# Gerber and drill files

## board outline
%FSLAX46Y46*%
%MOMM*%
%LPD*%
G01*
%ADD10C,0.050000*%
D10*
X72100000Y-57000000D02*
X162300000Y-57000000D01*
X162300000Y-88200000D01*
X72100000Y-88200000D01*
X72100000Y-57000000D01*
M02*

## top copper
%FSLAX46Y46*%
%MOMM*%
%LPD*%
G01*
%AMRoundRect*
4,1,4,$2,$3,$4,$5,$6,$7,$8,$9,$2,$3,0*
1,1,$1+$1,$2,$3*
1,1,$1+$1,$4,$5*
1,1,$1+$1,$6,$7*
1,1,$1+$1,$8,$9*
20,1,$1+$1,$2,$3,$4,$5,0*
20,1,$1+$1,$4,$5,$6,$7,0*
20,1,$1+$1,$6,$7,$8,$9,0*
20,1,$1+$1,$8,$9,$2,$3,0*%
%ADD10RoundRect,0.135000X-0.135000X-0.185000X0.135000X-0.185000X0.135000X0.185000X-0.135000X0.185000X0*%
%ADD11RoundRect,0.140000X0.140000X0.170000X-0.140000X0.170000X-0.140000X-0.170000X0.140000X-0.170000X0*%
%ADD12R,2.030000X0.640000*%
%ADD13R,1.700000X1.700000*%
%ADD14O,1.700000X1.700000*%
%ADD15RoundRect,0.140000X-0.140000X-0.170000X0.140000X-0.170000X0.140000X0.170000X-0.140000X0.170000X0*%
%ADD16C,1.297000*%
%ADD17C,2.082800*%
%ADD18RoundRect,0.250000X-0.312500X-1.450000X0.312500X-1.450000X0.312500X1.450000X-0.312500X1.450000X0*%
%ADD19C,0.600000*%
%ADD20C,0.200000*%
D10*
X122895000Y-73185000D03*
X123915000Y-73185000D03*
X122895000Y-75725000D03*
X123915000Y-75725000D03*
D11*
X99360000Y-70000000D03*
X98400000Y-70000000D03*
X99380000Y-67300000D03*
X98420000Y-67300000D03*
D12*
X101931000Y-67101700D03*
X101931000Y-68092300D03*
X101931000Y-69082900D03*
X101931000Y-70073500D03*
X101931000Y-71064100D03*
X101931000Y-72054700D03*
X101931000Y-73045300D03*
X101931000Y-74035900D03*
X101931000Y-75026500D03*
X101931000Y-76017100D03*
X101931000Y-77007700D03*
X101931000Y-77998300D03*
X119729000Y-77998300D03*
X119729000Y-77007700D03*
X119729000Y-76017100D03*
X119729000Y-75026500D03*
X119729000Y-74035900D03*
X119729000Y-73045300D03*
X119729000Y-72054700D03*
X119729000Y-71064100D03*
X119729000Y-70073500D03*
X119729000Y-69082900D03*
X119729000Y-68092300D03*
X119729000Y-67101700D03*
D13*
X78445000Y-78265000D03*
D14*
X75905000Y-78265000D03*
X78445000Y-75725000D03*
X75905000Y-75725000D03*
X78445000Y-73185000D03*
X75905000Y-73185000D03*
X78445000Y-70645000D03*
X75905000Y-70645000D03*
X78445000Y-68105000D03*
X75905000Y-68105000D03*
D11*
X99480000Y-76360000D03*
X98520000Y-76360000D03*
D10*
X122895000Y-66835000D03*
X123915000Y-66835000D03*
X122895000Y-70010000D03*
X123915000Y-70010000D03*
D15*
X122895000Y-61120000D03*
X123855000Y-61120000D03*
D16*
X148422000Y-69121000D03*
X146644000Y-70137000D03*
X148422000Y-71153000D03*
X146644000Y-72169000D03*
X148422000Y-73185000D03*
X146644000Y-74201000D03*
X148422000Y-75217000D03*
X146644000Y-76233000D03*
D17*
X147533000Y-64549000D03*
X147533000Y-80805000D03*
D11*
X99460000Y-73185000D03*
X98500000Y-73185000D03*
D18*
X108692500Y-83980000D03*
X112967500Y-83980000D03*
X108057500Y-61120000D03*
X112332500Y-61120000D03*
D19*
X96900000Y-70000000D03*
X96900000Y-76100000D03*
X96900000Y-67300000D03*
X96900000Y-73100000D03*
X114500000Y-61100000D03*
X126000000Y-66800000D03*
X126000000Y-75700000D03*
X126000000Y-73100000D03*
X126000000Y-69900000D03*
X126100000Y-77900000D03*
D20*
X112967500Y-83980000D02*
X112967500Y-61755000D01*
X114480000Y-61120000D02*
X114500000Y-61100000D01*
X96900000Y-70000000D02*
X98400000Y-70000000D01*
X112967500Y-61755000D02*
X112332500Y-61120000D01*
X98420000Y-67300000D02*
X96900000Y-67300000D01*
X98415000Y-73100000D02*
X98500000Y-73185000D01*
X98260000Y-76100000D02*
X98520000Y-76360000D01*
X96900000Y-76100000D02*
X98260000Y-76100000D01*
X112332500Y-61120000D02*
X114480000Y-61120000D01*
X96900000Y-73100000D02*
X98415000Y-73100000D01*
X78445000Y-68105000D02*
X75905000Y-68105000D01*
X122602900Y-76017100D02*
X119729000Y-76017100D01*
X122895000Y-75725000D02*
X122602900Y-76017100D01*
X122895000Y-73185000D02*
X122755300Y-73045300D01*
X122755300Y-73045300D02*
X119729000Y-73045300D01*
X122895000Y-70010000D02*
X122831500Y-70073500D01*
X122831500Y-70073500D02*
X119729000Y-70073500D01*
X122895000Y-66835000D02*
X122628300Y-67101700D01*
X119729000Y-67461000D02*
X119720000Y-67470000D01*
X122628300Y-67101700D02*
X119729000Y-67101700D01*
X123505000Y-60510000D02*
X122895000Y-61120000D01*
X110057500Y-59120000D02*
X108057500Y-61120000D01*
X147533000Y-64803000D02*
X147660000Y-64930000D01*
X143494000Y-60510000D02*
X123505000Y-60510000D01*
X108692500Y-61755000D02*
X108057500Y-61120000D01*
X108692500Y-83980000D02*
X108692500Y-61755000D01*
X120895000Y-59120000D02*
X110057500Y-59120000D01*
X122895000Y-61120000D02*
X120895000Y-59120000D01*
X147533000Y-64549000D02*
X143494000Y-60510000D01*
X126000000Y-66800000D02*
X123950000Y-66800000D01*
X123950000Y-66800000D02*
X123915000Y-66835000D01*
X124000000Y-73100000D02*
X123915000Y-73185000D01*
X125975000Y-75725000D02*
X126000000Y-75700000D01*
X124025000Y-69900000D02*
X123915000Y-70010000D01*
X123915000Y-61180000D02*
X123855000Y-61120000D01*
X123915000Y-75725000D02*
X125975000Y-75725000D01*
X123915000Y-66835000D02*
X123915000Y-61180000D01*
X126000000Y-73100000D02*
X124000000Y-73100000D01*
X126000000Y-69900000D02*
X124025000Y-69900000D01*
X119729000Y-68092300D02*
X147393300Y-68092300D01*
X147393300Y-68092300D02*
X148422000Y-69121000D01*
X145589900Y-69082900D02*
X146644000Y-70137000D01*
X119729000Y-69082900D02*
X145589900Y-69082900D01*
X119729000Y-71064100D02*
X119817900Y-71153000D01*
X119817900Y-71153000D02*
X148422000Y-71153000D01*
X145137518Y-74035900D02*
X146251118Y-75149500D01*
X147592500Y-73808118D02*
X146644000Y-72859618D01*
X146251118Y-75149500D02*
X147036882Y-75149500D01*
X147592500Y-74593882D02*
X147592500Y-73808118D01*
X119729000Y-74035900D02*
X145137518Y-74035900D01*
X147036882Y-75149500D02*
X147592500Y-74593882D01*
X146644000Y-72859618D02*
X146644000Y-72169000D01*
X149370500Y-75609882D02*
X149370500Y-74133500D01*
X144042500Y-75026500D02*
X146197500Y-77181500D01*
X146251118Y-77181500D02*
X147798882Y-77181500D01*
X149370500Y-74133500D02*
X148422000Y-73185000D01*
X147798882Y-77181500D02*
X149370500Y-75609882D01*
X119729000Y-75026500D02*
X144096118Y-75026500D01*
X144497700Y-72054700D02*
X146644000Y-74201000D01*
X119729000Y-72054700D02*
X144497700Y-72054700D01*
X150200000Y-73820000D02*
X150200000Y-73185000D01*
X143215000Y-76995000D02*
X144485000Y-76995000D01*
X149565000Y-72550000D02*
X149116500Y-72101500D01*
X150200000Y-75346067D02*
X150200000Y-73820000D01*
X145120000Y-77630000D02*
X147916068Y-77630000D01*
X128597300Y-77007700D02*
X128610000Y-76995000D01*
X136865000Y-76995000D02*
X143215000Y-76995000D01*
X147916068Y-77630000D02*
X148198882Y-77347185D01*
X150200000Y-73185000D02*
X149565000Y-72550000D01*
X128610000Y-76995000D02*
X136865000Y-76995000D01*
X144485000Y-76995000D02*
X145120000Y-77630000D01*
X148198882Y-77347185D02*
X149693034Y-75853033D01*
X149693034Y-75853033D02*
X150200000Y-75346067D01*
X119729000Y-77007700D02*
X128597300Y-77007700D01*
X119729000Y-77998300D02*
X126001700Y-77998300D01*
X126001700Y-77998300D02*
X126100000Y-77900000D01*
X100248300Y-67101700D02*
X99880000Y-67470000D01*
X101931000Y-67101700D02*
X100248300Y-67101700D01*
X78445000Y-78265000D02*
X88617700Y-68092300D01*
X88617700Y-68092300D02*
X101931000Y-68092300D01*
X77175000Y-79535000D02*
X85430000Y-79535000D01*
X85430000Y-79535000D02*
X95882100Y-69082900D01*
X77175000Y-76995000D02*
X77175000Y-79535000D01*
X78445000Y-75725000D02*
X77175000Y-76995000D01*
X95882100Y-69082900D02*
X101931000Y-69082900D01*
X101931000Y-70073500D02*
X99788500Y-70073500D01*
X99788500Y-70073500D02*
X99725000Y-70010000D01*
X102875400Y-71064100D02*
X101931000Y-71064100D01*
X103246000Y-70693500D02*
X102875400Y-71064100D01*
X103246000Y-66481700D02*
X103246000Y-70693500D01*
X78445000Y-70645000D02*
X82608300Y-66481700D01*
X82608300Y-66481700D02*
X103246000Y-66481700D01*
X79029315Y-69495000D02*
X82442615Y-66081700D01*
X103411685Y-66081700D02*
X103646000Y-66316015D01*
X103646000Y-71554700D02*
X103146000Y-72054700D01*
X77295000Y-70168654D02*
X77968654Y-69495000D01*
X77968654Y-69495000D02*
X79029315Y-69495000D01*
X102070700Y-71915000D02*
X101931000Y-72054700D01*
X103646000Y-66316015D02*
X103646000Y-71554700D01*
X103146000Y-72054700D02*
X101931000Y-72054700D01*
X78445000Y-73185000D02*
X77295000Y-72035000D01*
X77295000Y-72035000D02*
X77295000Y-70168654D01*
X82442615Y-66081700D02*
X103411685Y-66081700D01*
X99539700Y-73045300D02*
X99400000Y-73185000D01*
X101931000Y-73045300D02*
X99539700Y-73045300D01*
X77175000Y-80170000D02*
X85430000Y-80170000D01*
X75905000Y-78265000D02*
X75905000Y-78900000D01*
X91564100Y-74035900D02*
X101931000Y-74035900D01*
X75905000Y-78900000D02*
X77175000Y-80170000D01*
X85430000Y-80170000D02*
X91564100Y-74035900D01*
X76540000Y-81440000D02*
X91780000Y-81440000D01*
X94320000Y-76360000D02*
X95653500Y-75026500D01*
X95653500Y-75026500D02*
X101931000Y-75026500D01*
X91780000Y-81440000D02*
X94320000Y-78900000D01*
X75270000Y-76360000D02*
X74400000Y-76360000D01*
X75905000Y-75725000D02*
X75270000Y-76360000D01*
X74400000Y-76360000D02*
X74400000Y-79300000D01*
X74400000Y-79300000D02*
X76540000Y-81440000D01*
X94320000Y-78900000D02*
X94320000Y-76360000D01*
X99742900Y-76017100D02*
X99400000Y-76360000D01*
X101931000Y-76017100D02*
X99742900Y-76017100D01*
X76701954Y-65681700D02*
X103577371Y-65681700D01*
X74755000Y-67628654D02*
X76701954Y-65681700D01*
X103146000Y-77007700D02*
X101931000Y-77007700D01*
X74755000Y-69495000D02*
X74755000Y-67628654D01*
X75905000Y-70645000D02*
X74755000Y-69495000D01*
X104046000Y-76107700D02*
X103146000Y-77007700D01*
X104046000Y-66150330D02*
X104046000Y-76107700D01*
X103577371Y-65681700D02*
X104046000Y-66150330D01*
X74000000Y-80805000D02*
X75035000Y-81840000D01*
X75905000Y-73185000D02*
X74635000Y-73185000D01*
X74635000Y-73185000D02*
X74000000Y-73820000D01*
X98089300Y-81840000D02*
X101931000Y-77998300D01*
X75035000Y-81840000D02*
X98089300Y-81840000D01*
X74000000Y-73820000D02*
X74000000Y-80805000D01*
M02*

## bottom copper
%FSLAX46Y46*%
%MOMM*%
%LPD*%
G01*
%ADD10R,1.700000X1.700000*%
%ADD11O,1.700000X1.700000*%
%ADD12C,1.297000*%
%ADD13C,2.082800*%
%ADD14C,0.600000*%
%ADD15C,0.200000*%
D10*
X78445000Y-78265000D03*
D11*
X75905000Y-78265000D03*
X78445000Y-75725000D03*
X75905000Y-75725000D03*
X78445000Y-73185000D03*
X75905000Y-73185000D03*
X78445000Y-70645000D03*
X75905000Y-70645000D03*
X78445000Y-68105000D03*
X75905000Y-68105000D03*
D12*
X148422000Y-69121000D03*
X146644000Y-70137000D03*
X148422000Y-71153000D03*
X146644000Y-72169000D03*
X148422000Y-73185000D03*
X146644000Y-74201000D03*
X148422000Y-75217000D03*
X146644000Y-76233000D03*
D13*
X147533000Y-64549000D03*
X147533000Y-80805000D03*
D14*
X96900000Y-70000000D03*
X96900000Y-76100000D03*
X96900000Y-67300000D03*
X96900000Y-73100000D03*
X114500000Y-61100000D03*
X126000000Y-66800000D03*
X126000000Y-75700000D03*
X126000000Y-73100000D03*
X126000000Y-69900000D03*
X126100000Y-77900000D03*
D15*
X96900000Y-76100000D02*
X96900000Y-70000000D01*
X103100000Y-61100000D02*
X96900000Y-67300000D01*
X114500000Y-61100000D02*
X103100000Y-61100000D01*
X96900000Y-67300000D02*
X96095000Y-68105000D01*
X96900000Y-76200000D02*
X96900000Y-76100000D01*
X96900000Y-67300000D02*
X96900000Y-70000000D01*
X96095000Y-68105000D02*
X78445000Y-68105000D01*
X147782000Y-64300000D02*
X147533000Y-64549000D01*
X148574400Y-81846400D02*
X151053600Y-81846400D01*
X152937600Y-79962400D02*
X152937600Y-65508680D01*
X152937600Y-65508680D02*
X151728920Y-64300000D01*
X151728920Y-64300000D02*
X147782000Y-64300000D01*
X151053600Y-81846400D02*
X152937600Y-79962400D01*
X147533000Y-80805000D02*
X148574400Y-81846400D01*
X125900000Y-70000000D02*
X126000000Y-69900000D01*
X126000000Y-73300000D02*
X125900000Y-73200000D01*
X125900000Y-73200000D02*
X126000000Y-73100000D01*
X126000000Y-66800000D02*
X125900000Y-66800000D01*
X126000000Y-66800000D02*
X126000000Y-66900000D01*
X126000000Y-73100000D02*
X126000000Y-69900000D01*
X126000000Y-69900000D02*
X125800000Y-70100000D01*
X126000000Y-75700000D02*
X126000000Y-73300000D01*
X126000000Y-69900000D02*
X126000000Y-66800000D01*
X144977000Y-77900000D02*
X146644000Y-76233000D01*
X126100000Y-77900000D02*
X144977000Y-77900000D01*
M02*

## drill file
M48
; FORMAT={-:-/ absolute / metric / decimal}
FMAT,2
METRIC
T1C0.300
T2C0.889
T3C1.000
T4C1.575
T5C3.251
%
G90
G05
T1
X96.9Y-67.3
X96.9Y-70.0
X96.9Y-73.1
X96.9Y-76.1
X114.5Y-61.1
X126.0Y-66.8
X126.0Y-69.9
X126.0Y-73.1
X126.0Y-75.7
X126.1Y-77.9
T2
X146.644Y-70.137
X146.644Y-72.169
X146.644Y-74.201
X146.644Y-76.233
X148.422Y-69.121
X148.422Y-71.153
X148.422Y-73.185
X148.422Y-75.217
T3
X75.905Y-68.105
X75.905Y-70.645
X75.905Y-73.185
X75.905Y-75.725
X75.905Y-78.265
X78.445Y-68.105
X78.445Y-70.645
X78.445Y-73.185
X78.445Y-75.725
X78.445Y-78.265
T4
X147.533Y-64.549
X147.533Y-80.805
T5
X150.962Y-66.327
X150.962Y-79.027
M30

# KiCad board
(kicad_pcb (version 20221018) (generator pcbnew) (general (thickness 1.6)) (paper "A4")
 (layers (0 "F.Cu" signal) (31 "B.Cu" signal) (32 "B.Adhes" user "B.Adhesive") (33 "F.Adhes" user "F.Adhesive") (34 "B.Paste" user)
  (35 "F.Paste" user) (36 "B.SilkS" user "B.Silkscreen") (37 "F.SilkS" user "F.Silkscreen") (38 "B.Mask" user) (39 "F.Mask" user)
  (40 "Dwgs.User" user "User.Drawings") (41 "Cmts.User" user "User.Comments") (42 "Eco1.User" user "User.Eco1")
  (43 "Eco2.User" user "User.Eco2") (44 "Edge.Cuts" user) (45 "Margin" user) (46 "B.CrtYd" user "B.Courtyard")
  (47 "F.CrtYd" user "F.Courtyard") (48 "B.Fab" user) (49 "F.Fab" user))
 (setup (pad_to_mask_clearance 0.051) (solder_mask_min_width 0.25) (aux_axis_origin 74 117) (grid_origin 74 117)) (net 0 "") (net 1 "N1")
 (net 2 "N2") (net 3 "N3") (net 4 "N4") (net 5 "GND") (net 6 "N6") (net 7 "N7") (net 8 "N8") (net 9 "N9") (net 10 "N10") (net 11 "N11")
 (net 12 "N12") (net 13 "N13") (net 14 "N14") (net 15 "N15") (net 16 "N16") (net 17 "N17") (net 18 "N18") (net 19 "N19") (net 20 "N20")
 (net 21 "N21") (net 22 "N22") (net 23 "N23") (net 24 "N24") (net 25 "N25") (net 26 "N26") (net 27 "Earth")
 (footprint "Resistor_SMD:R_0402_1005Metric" (layer "F.Cu") (at 123.405 73.185)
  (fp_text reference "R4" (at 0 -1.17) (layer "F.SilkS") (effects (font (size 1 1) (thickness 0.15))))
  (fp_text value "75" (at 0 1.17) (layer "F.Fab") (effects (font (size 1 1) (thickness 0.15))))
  (pad "1" smd roundrect (at -0.51 0) (size 0.54 0.64) (layers "F.Cu" "F.Paste" "F.Mask") (roundrect_rratio 0.25) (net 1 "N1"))
  (pad "2" smd roundrect (at 0.51 0) (size 0.54 0.64) (layers "F.Cu" "F.Paste" "F.Mask") (roundrect_rratio 0.25) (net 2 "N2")))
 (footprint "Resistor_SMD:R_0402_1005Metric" (layer "F.Cu") (at 123.405 75.725)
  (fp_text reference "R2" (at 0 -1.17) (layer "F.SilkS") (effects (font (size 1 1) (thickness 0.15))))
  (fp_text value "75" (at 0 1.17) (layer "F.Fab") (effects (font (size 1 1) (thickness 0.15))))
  (pad "1" smd roundrect (at -0.51 0) (size 0.54 0.64) (layers "F.Cu" "F.Paste" "F.Mask") (roundrect_rratio 0.25) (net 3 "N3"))
  (pad "2" smd roundrect (at 0.51 0) (size 0.54 0.64) (layers "F.Cu" "F.Paste" "F.Mask") (roundrect_rratio 0.25) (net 2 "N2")))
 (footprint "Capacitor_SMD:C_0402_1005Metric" (layer "F.Cu") (at 98.88 70 180)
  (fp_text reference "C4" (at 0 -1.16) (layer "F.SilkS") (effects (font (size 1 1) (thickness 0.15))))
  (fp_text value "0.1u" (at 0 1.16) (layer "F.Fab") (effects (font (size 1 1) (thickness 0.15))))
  (pad "1" smd roundrect (at -0.48 0 180) (size 0.56 0.62) (layers "F.Cu" "F.Paste" "F.Mask") (roundrect_rratio 0.25) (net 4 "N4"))
  (pad "2" smd roundrect (at 0.48 0 180) (size 0.56 0.62) (layers "F.Cu" "F.Paste" "F.Mask") (roundrect_rratio 0.25) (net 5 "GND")))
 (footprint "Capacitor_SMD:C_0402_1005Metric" (layer "F.Cu") (at 98.9 67.3 180)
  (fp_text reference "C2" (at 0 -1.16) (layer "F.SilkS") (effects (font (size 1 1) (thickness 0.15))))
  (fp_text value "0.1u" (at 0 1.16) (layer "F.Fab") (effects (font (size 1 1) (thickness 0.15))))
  (pad "1" smd roundrect (at -0.48 0 180) (size 0.56 0.62) (layers "F.Cu" "F.Paste" "F.Mask") (roundrect_rratio 0.25) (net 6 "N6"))
  (pad "2" smd roundrect (at 0.48 0 180) (size 0.56 0.62) (layers "F.Cu" "F.Paste" "F.Mask") (roundrect_rratio 0.25) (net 5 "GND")))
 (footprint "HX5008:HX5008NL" (layer "F.Cu") (at 106.63 72.55)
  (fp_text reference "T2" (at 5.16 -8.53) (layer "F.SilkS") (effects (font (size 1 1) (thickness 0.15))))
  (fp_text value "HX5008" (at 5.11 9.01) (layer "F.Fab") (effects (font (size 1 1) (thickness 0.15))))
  (pad "1" smd rect (at -4.699 -5.4483 270) (size 0.64 2.03) (layers "F.Cu" "F.Paste" "F.Mask") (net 6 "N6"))
  (pad "2" smd rect (at -4.699 -4.4577 270) (size 0.64 2.03) (layers "F.Cu" "F.Paste" "F.Mask") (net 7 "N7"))
  (pad "3" smd rect (at -4.699 -3.4671 270) (size 0.64 2.03) (layers "F.Cu" "F.Paste" "F.Mask") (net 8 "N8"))
  (pad "4" smd rect (at -4.699 -2.4765 270) (size 0.64 2.03) (layers "F.Cu" "F.Paste" "F.Mask") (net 4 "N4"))
  (pad "5" smd rect (at -4.699 -1.4859 270) (size 0.64 2.03) (layers "F.Cu" "F.Paste" "F.Mask") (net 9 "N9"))
  (pad "6" smd rect (at -4.699 -0.4953 270) (size 0.64 2.03) (layers "F.Cu" "F.Paste" "F.Mask") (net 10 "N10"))
  (pad "7" smd rect (at -4.699 0.4953 270) (size 0.64 2.03) (layers "F.Cu" "F.Paste" "F.Mask") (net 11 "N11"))
  (pad "8" smd rect (at -4.699 1.4859 270) (size 0.64 2.03) (layers "F.Cu" "F.Paste" "F.Mask") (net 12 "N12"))
  (pad "9" smd rect (at -4.699 2.4765 270) (size 0.64 2.03) (layers "F.Cu" "F.Paste" "F.Mask") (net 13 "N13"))
  (pad "10" smd rect (at -4.699 3.4671 270) (size 0.64 2.03) (layers "F.Cu" "F.Paste" "F.Mask") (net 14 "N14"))
  (pad "11" smd rect (at -4.699 4.4577 270) (size 0.64 2.03) (layers "F.Cu" "F.Paste" "F.Mask") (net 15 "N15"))
  (pad "12" smd rect (at -4.699 5.4483 270) (size 0.64 2.03) (layers "F.Cu" "F.Paste" "F.Mask") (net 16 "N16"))
  (pad "13" smd rect (at 13.099 5.4483 270) (size 0.64 2.03) (layers "F.Cu" "F.Paste" "F.Mask") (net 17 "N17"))
  (pad "14" smd rect (at 13.099 4.4577 270) (size 0.64 2.03) (layers "F.Cu" "F.Paste" "F.Mask") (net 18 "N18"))
  (pad "15" smd rect (at 13.099 3.4671 270) (size 0.64 2.03) (layers "F.Cu" "F.Paste" "F.Mask") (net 3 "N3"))
  (pad "16" smd rect (at 13.099 2.4765 270) (size 0.64 2.03) (layers "F.Cu" "F.Paste" "F.Mask") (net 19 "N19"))
  (pad "17" smd rect (at 13.099 1.4859 270) (size 0.64 2.03) (layers "F.Cu" "F.Paste" "F.Mask") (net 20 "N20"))
  (pad "18" smd rect (at 13.099 0.4953 270) (size 0.64 2.03) (layers "F.Cu" "F.Paste" "F.Mask") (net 1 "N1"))
  (pad "19" smd rect (at 13.099 -0.4953 270) (size 0.64 2.03) (layers "F.Cu" "F.Paste" "F.Mask") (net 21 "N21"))
  (pad "20" smd rect (at 13.099 -1.4859 270) (size 0.64 2.03) (layers "F.Cu" "F.Paste" "F.Mask") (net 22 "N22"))
  (pad "21" smd rect (at 13.099 -2.4765 270) (size 0.64 2.03) (layers "F.Cu" "F.Paste" "F.Mask") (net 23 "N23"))
  (pad "22" smd rect (at 13.099 -3.4671 270) (size 0.64 2.03) (layers "F.Cu" "F.Paste" "F.Mask") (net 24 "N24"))
  (pad "23" smd rect (at 13.099 -4.4577 270) (size 0.64 2.03) (layers "F.Cu" "F.Paste" "F.Mask") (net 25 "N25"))
  (pad "24" smd rect (at 13.099 -5.4483 270) (size 0.64 2.03) (layers "F.Cu" "F.Paste" "F.Mask") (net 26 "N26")))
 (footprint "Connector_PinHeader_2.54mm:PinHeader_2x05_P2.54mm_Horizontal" (layer "F.Cu") (at 78.445 78.265 180)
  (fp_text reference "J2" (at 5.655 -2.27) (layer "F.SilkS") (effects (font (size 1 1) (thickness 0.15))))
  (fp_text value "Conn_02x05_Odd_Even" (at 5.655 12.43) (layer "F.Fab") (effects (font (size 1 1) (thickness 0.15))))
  (pad "1" thru_hole rect (at 0 0 180) (size 1.7 1.7) (drill 1) (layers "*.Cu" "*.Mask") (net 7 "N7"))
  (pad "2" thru_hole oval (at 2.54 0 180) (size 1.7 1.7) (drill 1) (layers "*.Cu" "*.Mask") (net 12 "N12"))
  (pad "3" thru_hole oval (at 0 2.54 180) (size 1.7 1.7) (drill 1) (layers "*.Cu" "*.Mask") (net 8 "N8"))
  (pad "4" thru_hole oval (at 2.54 2.54 180) (size 1.7 1.7) (drill 1) (layers "*.Cu" "*.Mask") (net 13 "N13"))
  (pad "5" thru_hole oval (at 0 5.08 180) (size 1.7 1.7) (drill 1) (layers "*.Cu" "*.Mask") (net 10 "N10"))
  (pad "6" thru_hole oval (at 2.54 5.08 180) (size 1.7 1.7) (drill 1) (layers "*.Cu" "*.Mask") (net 16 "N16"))
  (pad "7" thru_hole oval (at 0 7.62 180) (size 1.7 1.7) (drill 1) (layers "*.Cu" "*.Mask") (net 9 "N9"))
  (pad "8" thru_hole oval (at 2.54 7.62 180) (size 1.7 1.7) (drill 1) (layers "*.Cu" "*.Mask") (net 15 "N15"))
  (pad "9" thru_hole oval (at 0 10.16 180) (size 1.7 1.7) (drill 1) (layers "*.Cu" "*.Mask") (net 5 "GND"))
  (pad "10" thru_hole oval (at 2.54 10.16 180) (size 1.7 1.7) (drill 1) (layers "*.Cu" "*.Mask") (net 5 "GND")))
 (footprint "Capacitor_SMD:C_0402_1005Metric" (layer "F.Cu") (at 99 76.36 180)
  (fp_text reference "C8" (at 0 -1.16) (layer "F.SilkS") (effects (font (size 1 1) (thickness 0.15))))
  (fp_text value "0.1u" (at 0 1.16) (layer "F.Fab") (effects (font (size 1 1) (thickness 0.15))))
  (pad "1" smd roundrect (at -0.48 0 180) (size 0.56 0.62) (layers "F.Cu" "F.Paste" "F.Mask") (roundrect_rratio 0.25) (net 14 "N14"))
  (pad "2" smd roundrect (at 0.48 0 180) (size 0.56 0.62) (layers "F.Cu" "F.Paste" "F.Mask") (roundrect_rratio 0.25) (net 5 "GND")))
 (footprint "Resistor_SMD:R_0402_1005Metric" (layer "F.Cu") (at 123.405 66.835)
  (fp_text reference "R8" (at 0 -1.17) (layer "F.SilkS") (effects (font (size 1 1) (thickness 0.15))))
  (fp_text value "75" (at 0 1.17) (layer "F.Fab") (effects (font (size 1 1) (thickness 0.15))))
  (pad "1" smd roundrect (at -0.51 0) (size 0.54 0.64) (layers "F.Cu" "F.Paste" "F.Mask") (roundrect_rratio 0.25) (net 26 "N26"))
  (pad "2" smd roundrect (at 0.51 0) (size 0.54 0.64) (layers "F.Cu" "F.Paste" "F.Mask") (roundrect_rratio 0.25) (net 2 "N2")))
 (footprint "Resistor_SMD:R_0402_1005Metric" (layer "F.Cu") (at 123.405 70.01)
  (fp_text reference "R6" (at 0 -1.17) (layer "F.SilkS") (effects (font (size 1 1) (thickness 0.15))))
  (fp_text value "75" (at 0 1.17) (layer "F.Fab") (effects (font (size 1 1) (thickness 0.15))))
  (pad "1" smd roundrect (at -0.51 0) (size 0.54 0.64) (layers "F.Cu" "F.Paste" "F.Mask") (roundrect_rratio 0.25) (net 23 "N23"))
  (pad "2" smd roundrect (at 0.51 0) (size 0.54 0.64) (layers "F.Cu" "F.Paste" "F.Mask") (roundrect_rratio 0.25) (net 2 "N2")))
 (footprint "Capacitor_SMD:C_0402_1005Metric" (layer "F.Cu") (at 123.375 61.12)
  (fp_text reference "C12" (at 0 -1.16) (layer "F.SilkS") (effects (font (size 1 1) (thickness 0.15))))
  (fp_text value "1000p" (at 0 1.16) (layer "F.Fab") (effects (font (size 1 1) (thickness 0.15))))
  (pad "1" smd roundrect (at -0.48 0) (size 0.56 0.62) (layers "F.Cu" "F.Paste" "F.Mask") (roundrect_rratio 0.25) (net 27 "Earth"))
  (pad "2" smd roundrect (at 0.48 0) (size 0.56 0.62) (layers "F.Cu" "F.Paste" "F.Mask") (roundrect_rratio 0.25) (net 2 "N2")))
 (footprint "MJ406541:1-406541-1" (layer "F.Cu") (at 148.422 69.121 -90)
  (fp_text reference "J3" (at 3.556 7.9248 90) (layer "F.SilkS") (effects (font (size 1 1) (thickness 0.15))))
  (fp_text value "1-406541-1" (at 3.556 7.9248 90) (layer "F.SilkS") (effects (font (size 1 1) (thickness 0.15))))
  (pad "" np_thru_hole circle (at -2.794 -2.54 270) (size 3.2512 3.2512) (drill 3.2512) (layers "*.Cu" "*.Mask"))
  (pad "" np_thru_hole circle (at 9.906 -2.54 270) (size 3.2512 3.2512) (drill 3.2512) (layers "*.Cu" "*.Mask"))
  (pad "1" thru_hole circle (at 0 0 270) (size 1.297 1.297) (drill 0.889) (layers "*.Cu" "*.Mask") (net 25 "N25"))
  (pad "2" thru_hole circle (at 1.016 1.778 270) (size 1.297 1.297) (drill 0.889) (layers "*.Cu" "*.Mask") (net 24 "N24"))
  (pad "3" thru_hole circle (at 2.032 0 270) (size 1.297 1.297) (drill 0.889) (layers "*.Cu" "*.Mask") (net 22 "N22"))
  (pad "4" thru_hole circle (at 3.048 1.778 270) (size 1.297 1.297) (drill 0.889) (layers "*.Cu" "*.Mask") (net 20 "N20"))
  (pad "5" thru_hole circle (at 4.064 0 270) (size 1.297 1.297) (drill 0.889) (layers "*.Cu" "*.Mask") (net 19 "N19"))
  (pad "6" thru_hole circle (at 5.08 1.778 270) (size 1.297 1.297) (drill 0.889) (layers "*.Cu" "*.Mask") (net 21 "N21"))
  (pad "7" thru_hole circle (at 6.096 0 270) (size 1.297 1.297) (drill 0.889) (layers "*.Cu" "*.Mask") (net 18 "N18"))
  (pad "8" thru_hole circle (at 7.112 1.778 270) (size 1.297 1.297) (drill 0.889) (layers "*.Cu" "*.Mask") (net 17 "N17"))
  (pad "9" thru_hole circle (at -4.572 0.889 270) (size 2.0828 2.0828) (drill 1.5748) (layers "*.Cu" "*.Mask") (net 27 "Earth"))
  (pad "10" thru_hole circle (at 11.684 0.889 270) (size 2.0828 2.0828) (drill 1.5748) (layers "*.Cu" "*.Mask") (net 27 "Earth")))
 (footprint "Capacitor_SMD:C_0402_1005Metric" (layer "F.Cu") (at 98.98 73.185 180)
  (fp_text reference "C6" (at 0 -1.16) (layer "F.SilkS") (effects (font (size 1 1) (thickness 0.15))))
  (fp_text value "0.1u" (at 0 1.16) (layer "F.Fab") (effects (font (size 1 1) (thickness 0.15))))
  (pad "1" smd roundrect (at -0.48 0 180) (size 0.56 0.62) (layers "F.Cu" "F.Paste" "F.Mask") (roundrect_rratio 0.25) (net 11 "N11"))
  (pad "2" smd roundrect (at 0.48 0 180) (size 0.56 0.62) (layers "F.Cu" "F.Paste" "F.Mask") (roundrect_rratio 0.25) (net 5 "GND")))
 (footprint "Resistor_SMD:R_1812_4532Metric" (layer "F.Cu") (at 110.83 83.98)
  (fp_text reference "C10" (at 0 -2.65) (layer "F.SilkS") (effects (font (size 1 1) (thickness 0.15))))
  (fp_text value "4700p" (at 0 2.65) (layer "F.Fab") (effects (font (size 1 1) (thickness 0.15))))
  (pad "1" smd roundrect (at -2.1375 0) (size 1.125 3.4) (layers "F.Cu" "F.Paste" "F.Mask") (roundrect_rratio 0.222222) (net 27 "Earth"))
  (pad "2" smd roundrect (at 2.1375 0) (size 1.125 3.4) (layers "F.Cu" "F.Paste" "F.Mask") (roundrect_rratio 0.222222) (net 5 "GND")))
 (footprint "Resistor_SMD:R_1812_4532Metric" (layer "F.Cu") (at 110.195 61.12)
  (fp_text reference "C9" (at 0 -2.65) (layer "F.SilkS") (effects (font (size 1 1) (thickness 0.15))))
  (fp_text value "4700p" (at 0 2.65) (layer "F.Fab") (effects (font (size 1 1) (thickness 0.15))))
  (pad "1" smd roundrect (at -2.1375 0) (size 1.125 3.4) (layers "F.Cu" "F.Paste" "F.Mask") (roundrect_rratio 0.222222) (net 27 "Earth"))
  (pad "2" smd roundrect (at 2.1375 0) (size 1.125 3.4) (layers "F.Cu" "F.Paste" "F.Mask") (roundrect_rratio 0.222222) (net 5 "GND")))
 (gr_rect (start 72.1 57) (end 162.3 88.2) (stroke (width 0.05) (type default)) (fill none) (layer "Edge.Cuts"))
 (segment (start 112.9675 83.98) (end 112.9675 61.755) (width 0.2) (layer "F.Cu") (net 5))
 (segment (start 114.48 61.12) (end 114.5 61.1) (width 0.2) (layer "F.Cu") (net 5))
 (segment (start 96.9 70) (end 98.4 70) (width 0.2) (layer "F.Cu") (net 5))
 (segment (start 112.9675 61.755) (end 112.3325 61.12) (width 0.2) (layer "F.Cu") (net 5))
 (segment (start 98.42 67.3) (end 96.9 67.3) (width 0.2) (layer "F.Cu") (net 5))
 (segment (start 98.415 73.1) (end 98.5 73.185) (width 0.2) (layer "F.Cu") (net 5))
 (segment (start 98.26 76.1) (end 98.52 76.36) (width 0.2) (layer "F.Cu") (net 5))
 (segment (start 96.9 76.1) (end 98.26 76.1) (width 0.2) (layer "F.Cu") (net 5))
 (segment (start 112.3325 61.12) (end 114.48 61.12) (width 0.2) (layer "F.Cu") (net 5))
 (segment (start 96.9 73.1) (end 98.415 73.1) (width 0.2) (layer "F.Cu") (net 5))
 (segment (start 78.445 68.105) (end 75.905 68.105) (width 0.2) (layer "F.Cu") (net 5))
 (via (at 96.9 70) (size 0.6) (drill 0.3) (layers "F.Cu" "B.Cu") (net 5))
 (via (at 96.9 76.1) (size 0.6) (drill 0.3) (layers "F.Cu" "B.Cu") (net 5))
 (via (at 96.9 67.3) (size 0.6) (drill 0.3) (layers "F.Cu" "B.Cu") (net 5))
 (via (at 96.9 73.1) (size 0.6) (drill 0.3) (layers "F.Cu" "B.Cu") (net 5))
 (via (at 114.5 61.1) (size 0.6) (drill 0.3) (layers "F.Cu" "B.Cu") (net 5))
 (segment (start 96.9 76.1) (end 96.9 70) (width 0.2) (layer "B.Cu") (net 5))
 (segment (start 103.1 61.1) (end 96.9 67.3) (width 0.2) (layer "B.Cu") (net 5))
 (segment (start 114.5 61.1) (end 103.1 61.1) (width 0.2) (layer "B.Cu") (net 5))
 (segment (start 96.9 67.3) (end 96.095 68.105) (width 0.2) (layer "B.Cu") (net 5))
 (segment (start 96.9 76.2) (end 96.9 76.1) (width 0.2) (layer "B.Cu") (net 5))
 (segment (start 96.9 67.3) (end 96.9 70) (width 0.2) (layer "B.Cu") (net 5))
 (segment (start 96.095 68.105) (end 78.445 68.105) (width 0.2) (layer "B.Cu") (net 5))
 (segment (start 122.6029 76.0171) (end 119.729 76.0171) (width 0.2) (layer "F.Cu") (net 3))
 (segment (start 122.895 75.725) (end 122.6029 76.0171) (width 0.2) (layer "F.Cu") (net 3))
 (segment (start 122.895 73.185) (end 122.7553 73.0453) (width 0.2) (layer "F.Cu") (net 1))
 (segment (start 122.7553 73.0453) (end 119.729 73.0453) (width 0.2) (layer "F.Cu") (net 1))
 (segment (start 122.895 70.01) (end 122.8315 70.0735) (width 0.2) (layer "F.Cu") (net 23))
 (segment (start 122.8315 70.0735) (end 119.729 70.0735) (width 0.2) (layer "F.Cu") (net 23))
 (segment (start 122.895 66.835) (end 122.6283 67.1017) (width 0.2) (layer "F.Cu") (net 26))
 (segment (start 119.729 67.461) (end 119.72 67.47) (width 0.2) (layer "F.Cu") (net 26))
 (segment (start 122.6283 67.1017) (end 119.729 67.1017) (width 0.2) (layer "F.Cu") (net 26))
 (segment (start 123.505 60.51) (end 122.895 61.12) (width 0.2) (layer "F.Cu") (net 27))
 (segment (start 110.0575 59.12) (end 108.0575 61.12) (width 0.2) (layer "F.Cu") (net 27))
 (segment (start 147.533 64.803) (end 147.66 64.93) (width 0.2) (layer "F.Cu") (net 27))
 (segment (start 143.494 60.51) (end 123.505 60.51) (width 0.2) (layer "F.Cu") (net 27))
 (segment (start 108.6925 61.755) (end 108.0575 61.12) (width 0.2) (layer "F.Cu") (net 27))
 (segment (start 108.6925 83.98) (end 108.6925 61.755) (width 0.2) (layer "F.Cu") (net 27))
 (segment (start 120.895 59.12) (end 110.0575 59.12) (width 0.2) (layer "F.Cu") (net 27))
 (segment (start 122.895 61.12) (end 120.895 59.12) (width 0.2) (layer "F.Cu") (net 27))
 (segment (start 147.533 64.549) (end 143.494 60.51) (width 0.2) (layer "F.Cu") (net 27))
 (segment (start 147.782 64.3) (end 147.533 64.549) (width 0.2) (layer "B.Cu") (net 27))
 (segment (start 148.5744 81.8464) (end 151.0536 81.8464) (width 0.2) (layer "B.Cu") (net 27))
 (segment (start 152.9376 79.9624) (end 152.9376 65.50868) (width 0.2) (layer "B.Cu") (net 27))
 (segment (start 152.9376 65.50868) (end 151.72892 64.3) (width 0.2) (layer "B.Cu") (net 27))
 (segment (start 151.72892 64.3) (end 147.782 64.3) (width 0.2) (layer "B.Cu") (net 27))
 (segment (start 151.0536 81.8464) (end 152.9376 79.9624) (width 0.2) (layer "B.Cu") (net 27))
 (segment (start 147.533 80.805) (end 148.5744 81.8464) (width 0.2) (layer "B.Cu") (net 27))
 (segment (start 126 66.8) (end 123.95 66.8) (width 0.2) (layer "F.Cu") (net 2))
 (segment (start 123.95 66.8) (end 123.915 66.835) (width 0.2) (layer "F.Cu") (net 2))
 (segment (start 124 73.1) (end 123.915 73.185) (width 0.2) (layer "F.Cu") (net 2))
 (segment (start 125.975 75.725) (end 126 75.7) (width 0.2) (layer "F.Cu") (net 2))
 (segment (start 124.025 69.9) (end 123.915 70.01) (width 0.2) (layer "F.Cu") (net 2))
 (segment (start 123.915 61.18) (end 123.855 61.12) (width 0.2) (layer "F.Cu") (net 2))
 (segment (start 123.915 75.725) (end 125.975 75.725) (width 0.2) (layer "F.Cu") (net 2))
 (segment (start 123.915 66.835) (end 123.915 61.18) (width 0.2) (layer "F.Cu") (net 2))
 (segment (start 126 73.1) (end 124 73.1) (width 0.2) (layer "F.Cu") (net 2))
 (segment (start 126 69.9) (end 124.025 69.9) (width 0.2) (layer "F.Cu") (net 2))
 (via (at 126 66.8) (size 0.6) (drill 0.3) (layers "F.Cu" "B.Cu") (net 2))
 (via (at 126 75.7) (size 0.6) (drill 0.3) (layers "F.Cu" "B.Cu") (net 2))
 (via (at 126 73.1) (size 0.6) (drill 0.3) (layers "F.Cu" "B.Cu") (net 2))
 (via (at 126 69.9) (size 0.6) (drill 0.3) (layers "F.Cu" "B.Cu") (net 2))
 (segment (start 125.9 70) (end 126 69.9) (width 0.2) (layer "B.Cu") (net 2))
 (segment (start 126 73.3) (end 125.9 73.2) (width 0.2) (layer "B.Cu") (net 2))
 (segment (start 125.9 73.2) (end 126 73.1) (width 0.2) (layer "B.Cu") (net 2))
 (segment (start 126 66.8) (end 125.9 66.8) (width 0.2) (layer "B.Cu") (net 2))
 (segment (start 126 66.8) (end 126 66.9) (width 0.2) (layer "B.Cu") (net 2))
 (segment (start 126 73.1) (end 126 69.9) (width 0.2) (layer "B.Cu") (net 2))
 (segment (start 126 69.9) (end 125.8 70.1) (width 0.2) (layer "B.Cu") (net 2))
 (segment (start 126 75.7) (end 126 73.3) (width 0.2) (layer "B.Cu") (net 2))
 (segment (start 126 69.9) (end 126 66.8) (width 0.2) (layer "B.Cu") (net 2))
 (segment (start 119.729 68.0923) (end 147.3933 68.0923) (width 0.2) (layer "F.Cu") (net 25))
 (segment (start 147.3933 68.0923) (end 148.422 69.121) (width 0.2) (layer "F.Cu") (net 25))
 (segment (start 145.5899 69.0829) (end 146.644 70.137) (width 0.2) (layer "F.Cu") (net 24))
 (segment (start 119.729 69.0829) (end 145.5899 69.0829) (width 0.2) (layer "F.Cu") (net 24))
 (segment (start 119.729 71.0641) (end 119.8179 71.153) (width 0.2) (layer "F.Cu") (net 22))
 (segment (start 119.8179 71.153) (end 148.422 71.153) (width 0.2) (layer "F.Cu") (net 22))
 (segment (start 145.137518 74.0359) (end 146.251118 75.1495) (width 0.2) (layer "F.Cu") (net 20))
 (segment (start 147.5925 73.808118) (end 146.644 72.859618) (width 0.2) (layer "F.Cu") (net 20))
 (segment (start 146.251118 75.1495) (end 147.036882 75.1495) (width 0.2) (layer "F.Cu") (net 20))
 (segment (start 147.5925 74.593882) (end 147.5925 73.808118) (width 0.2) (layer "F.Cu") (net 20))
 (segment (start 119.729 74.0359) (end 145.137518 74.0359) (width 0.2) (layer "F.Cu") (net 20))
 (segment (start 147.036882 75.1495) (end 147.5925 74.593882) (width 0.2) (layer "F.Cu") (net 20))
 (segment (start 146.644 72.859618) (end 146.644 72.169) (width 0.2) (layer "F.Cu") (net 20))
 (segment (start 149.3705 75.609882) (end 149.3705 74.1335) (width 0.2) (layer "F.Cu") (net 19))
 (segment (start 144.0425 75.0265) (end 146.1975 77.1815) (width 0.2) (layer "F.Cu") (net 19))
 (segment (start 146.251118 77.1815) (end 147.798882 77.1815) (width 0.2) (layer "F.Cu") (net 19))
 (segment (start 149.3705 74.1335) (end 148.422 73.185) (width 0.2) (layer "F.Cu") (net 19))
 (segment (start 147.798882 77.1815) (end 149.3705 75.609882) (width 0.2) (layer "F.Cu") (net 19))
 (segment (start 119.729 75.0265) (end 144.096118 75.0265) (width 0.2) (layer "F.Cu") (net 19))
 (segment (start 144.4977 72.0547) (end 146.644 74.201) (width 0.2) (layer "F.Cu") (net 21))
 (segment (start 119.729 72.0547) (end 144.4977 72.0547) (width 0.2) (layer "F.Cu") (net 21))
 (segment (start 150.2 73.82) (end 150.2 73.185) (width 0.2) (layer "F.Cu") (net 18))
 (segment (start 143.215 76.995) (end 144.485 76.995) (width 0.2) (layer "F.Cu") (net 18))
 (segment (start 149.565 72.55) (end 149.1165 72.1015) (width 0.2) (layer "F.Cu") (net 18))
 (segment (start 150.2 75.346067) (end 150.2 73.82) (width 0.2) (layer "F.Cu") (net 18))
 (segment (start 145.12 77.63) (end 147.916068 77.63) (width 0.2) (layer "F.Cu") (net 18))
 (segment (start 128.5973 77.0077) (end 128.61 76.995) (width 0.2) (layer "F.Cu") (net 18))
 (segment (start 136.865 76.995) (end 143.215 76.995) (width 0.2) (layer "F.Cu") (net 18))
 (segment (start 147.916068 77.63) (end 148.198882 77.347185) (width 0.2) (layer "F.Cu") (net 18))
 (segment (start 150.2 73.185) (end 149.565 72.55) (width 0.2) (layer "F.Cu") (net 18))
 (segment (start 128.61 76.995) (end 136.865 76.995) (width 0.2) (layer "F.Cu") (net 18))
 (segment (start 144.485 76.995) (end 145.12 77.63) (width 0.2) (layer "F.Cu") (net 18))
 (segment (start 148.198882 77.347185) (end 149.693034 75.853033) (width 0.2) (layer "F.Cu") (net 18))
 (segment (start 149.693034 75.853033) (end 150.2 75.346067) (width 0.2) (layer "F.Cu") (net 18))
 (segment (start 119.729 77.0077) (end 128.5973 77.0077) (width 0.2) (layer "F.Cu") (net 18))
 (segment (start 119.729 77.9983) (end 126.0017 77.9983) (width 0.2) (layer "F.Cu") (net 17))
 (segment (start 126.0017 77.9983) (end 126.1 77.9) (width 0.2) (layer "F.Cu") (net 17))
 (via (at 126.1 77.9) (size 0.6) (drill 0.3) (layers "F.Cu" "B.Cu") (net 17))
 (segment (start 144.977 77.9) (end 146.644 76.233) (width 0.2) (layer "B.Cu") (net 17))
 (segment (start 126.1 77.9) (end 144.977 77.9) (width 0.2) (layer "B.Cu") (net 17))
 (segment (start 100.2483 67.1017) (end 99.88 67.47) (width 0.2) (layer "F.Cu") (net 6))
 (segment (start 101.931 67.1017) (end 100.2483 67.1017) (width 0.2) (layer "F.Cu") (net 6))
 (segment (start 78.445 78.265) (end 88.6177 68.0923) (width 0.2) (layer "F.Cu") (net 7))
 (segment (start 88.6177 68.0923) (end 101.931 68.0923) (width 0.2) (layer "F.Cu") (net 7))
 (segment (start 77.175 79.535) (end 85.43 79.535) (width 0.2) (layer "F.Cu") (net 8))
 (segment (start 85.43 79.535) (end 95.8821 69.0829) (width 0.2) (layer "F.Cu") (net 8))
 (segment (start 77.175 76.995) (end 77.175 79.535) (width 0.2) (layer "F.Cu") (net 8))
 (segment (start 78.445 75.725) (end 77.175 76.995) (width 0.2) (layer "F.Cu") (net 8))
 (segment (start 95.8821 69.0829) (end 101.931 69.0829) (width 0.2) (layer "F.Cu") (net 8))
 (segment (start 101.931 70.0735) (end 99.7885 70.0735) (width 0.2) (layer "F.Cu") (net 4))
 (segment (start 99.7885 70.0735) (end 99.725 70.01) (width 0.2) (layer "F.Cu") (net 4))
 (segment (start 102.8754 71.0641) (end 101.931 71.0641) (width 0.2) (layer "F.Cu") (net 9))
 (segment (start 103.246 70.6935) (end 102.8754 71.0641) (width 0.2) (layer "F.Cu") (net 9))
 (segment (start 103.246 66.4817) (end 103.246 70.6935) (width 0.2) (layer "F.Cu") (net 9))
 (segment (start 78.445 70.645) (end 82.6083 66.4817) (width 0.2) (layer "F.Cu") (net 9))
 (segment (start 82.6083 66.4817) (end 103.246 66.4817) (width 0.2) (layer "F.Cu") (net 9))
 (segment (start 79.029315 69.495) (end 82.442615 66.0817) (width 0.2) (layer "F.Cu") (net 10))
 (segment (start 103.411685 66.0817) (end 103.646 66.316015) (width 0.2) (layer "F.Cu") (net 10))
 (segment (start 103.646 71.5547) (end 103.146 72.0547) (width 0.2) (layer "F.Cu") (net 10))
 (segment (start 77.295 70.168654) (end 77.968654 69.495) (width 0.2) (layer "F.Cu") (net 10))
 (segment (start 77.968654 69.495) (end 79.029315 69.495) (width 0.2) (layer "F.Cu") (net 10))
 (segment (start 102.0707 71.915) (end 101.931 72.0547) (width 0.2) (layer "F.Cu") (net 10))
 (segment (start 103.646 66.316015) (end 103.646 71.5547) (width 0.2) (layer "F.Cu") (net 10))
 (segment (start 103.146 72.0547) (end 101.931 72.0547) (width 0.2) (layer "F.Cu") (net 10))
 (segment (start 78.445 73.185) (end 77.295 72.035) (width 0.2) (layer "F.Cu") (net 10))
 (segment (start 77.295 72.035) (end 77.295 70.168654) (width 0.2) (layer "F.Cu") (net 10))
 (segment (start 82.442615 66.0817) (end 103.411685 66.0817) (width 0.2) (layer "F.Cu") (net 10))
 (segment (start 99.5397 73.0453) (end 99.4 73.185) (width 0.2) (layer "F.Cu") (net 11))
 (segment (start 101.931 73.0453) (end 99.5397 73.0453) (width 0.2) (layer "F.Cu") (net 11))
 (segment (start 77.175 80.17) (end 85.43 80.17) (width 0.2) (layer "F.Cu") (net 12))
 (segment (start 75.905 78.265) (end 75.905 78.9) (width 0.2) (layer "F.Cu") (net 12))
 (segment (start 91.5641 74.0359) (end 101.931 74.0359) (width 0.2) (layer "F.Cu") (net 12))
 (segment (start 75.905 78.9) (end 77.175 80.17) (width 0.2) (layer "F.Cu") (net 12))
 (segment (start 85.43 80.17) (end 91.5641 74.0359) (width 0.2) (layer "F.Cu") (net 12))
 (segment (start 76.54 81.44) (end 91.78 81.44) (width 0.2) (layer "F.Cu") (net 13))
 (segment (start 94.32 76.36) (end 95.6535 75.0265) (width 0.2) (layer "F.Cu") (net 13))
 (segment (start 95.6535 75.0265) (end 101.931 75.0265) (width 0.2) (layer "F.Cu") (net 13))
 (segment (start 91.78 81.44) (end 94.32 78.9) (width 0.2) (layer "F.Cu") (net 13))
 (segment (start 75.27 76.36) (end 74.4 76.36) (width 0.2) (layer "F.Cu") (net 13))
 (segment (start 75.905 75.725) (end 75.27 76.36) (width 0.2) (layer "F.Cu") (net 13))
 (segment (start 74.4 76.36) (end 74.4 79.3) (width 0.2) (layer "F.Cu") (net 13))
 (segment (start 74.4 79.3) (end 76.54 81.44) (width 0.2) (layer "F.Cu") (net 13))
 (segment (start 94.32 78.9) (end 94.32 76.36) (width 0.2) (layer "F.Cu") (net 13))
 (segment (start 99.7429 76.0171) (end 99.4 76.36) (width 0.2) (layer "F.Cu") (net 14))
 (segment (start 101.931 76.0171) (end 99.7429 76.0171) (width 0.2) (layer "F.Cu") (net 14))
 (segment (start 76.701954 65.6817) (end 103.577371 65.6817) (width 0.2) (layer "F.Cu") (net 15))
 (segment (start 74.755 67.628654) (end 76.701954 65.6817) (width 0.2) (layer "F.Cu") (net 15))
 (segment (start 103.146 77.0077) (end 101.931 77.0077) (width 0.2) (layer "F.Cu") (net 15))
 (segment (start 74.755 69.495) (end 74.755 67.628654) (width 0.2) (layer "F.Cu") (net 15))
 (segment (start 75.905 70.645) (end 74.755 69.495) (width 0.2) (layer "F.Cu") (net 15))
 (segment (start 104.046 76.1077) (end 103.146 77.0077) (width 0.2) (layer "F.Cu") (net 15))
 (segment (start 104.046 66.15033) (end 104.046 76.1077) (width 0.2) (layer "F.Cu") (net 15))
 (segment (start 103.577371 65.6817) (end 104.046 66.15033) (width 0.2) (layer "F.Cu") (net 15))
 (segment (start 74 80.805) (end 75.035 81.84) (width 0.2) (layer "F.Cu") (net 16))
 (segment (start 75.905 73.185) (end 74.635 73.185) (width 0.2) (layer "F.Cu") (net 16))
 (segment (start 74.635 73.185) (end 74 73.82) (width 0.2) (layer "F.Cu") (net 16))
 (segment (start 98.0893 81.84) (end 101.931 77.9983) (width 0.2) (layer "F.Cu") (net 16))
 (segment (start 75.035 81.84) (end 98.0893 81.84) (width 0.2) (layer "F.Cu") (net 16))
 (segment (start 74 73.82) (end 74 80.805) (width 0.2) (layer "F.Cu") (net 16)))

